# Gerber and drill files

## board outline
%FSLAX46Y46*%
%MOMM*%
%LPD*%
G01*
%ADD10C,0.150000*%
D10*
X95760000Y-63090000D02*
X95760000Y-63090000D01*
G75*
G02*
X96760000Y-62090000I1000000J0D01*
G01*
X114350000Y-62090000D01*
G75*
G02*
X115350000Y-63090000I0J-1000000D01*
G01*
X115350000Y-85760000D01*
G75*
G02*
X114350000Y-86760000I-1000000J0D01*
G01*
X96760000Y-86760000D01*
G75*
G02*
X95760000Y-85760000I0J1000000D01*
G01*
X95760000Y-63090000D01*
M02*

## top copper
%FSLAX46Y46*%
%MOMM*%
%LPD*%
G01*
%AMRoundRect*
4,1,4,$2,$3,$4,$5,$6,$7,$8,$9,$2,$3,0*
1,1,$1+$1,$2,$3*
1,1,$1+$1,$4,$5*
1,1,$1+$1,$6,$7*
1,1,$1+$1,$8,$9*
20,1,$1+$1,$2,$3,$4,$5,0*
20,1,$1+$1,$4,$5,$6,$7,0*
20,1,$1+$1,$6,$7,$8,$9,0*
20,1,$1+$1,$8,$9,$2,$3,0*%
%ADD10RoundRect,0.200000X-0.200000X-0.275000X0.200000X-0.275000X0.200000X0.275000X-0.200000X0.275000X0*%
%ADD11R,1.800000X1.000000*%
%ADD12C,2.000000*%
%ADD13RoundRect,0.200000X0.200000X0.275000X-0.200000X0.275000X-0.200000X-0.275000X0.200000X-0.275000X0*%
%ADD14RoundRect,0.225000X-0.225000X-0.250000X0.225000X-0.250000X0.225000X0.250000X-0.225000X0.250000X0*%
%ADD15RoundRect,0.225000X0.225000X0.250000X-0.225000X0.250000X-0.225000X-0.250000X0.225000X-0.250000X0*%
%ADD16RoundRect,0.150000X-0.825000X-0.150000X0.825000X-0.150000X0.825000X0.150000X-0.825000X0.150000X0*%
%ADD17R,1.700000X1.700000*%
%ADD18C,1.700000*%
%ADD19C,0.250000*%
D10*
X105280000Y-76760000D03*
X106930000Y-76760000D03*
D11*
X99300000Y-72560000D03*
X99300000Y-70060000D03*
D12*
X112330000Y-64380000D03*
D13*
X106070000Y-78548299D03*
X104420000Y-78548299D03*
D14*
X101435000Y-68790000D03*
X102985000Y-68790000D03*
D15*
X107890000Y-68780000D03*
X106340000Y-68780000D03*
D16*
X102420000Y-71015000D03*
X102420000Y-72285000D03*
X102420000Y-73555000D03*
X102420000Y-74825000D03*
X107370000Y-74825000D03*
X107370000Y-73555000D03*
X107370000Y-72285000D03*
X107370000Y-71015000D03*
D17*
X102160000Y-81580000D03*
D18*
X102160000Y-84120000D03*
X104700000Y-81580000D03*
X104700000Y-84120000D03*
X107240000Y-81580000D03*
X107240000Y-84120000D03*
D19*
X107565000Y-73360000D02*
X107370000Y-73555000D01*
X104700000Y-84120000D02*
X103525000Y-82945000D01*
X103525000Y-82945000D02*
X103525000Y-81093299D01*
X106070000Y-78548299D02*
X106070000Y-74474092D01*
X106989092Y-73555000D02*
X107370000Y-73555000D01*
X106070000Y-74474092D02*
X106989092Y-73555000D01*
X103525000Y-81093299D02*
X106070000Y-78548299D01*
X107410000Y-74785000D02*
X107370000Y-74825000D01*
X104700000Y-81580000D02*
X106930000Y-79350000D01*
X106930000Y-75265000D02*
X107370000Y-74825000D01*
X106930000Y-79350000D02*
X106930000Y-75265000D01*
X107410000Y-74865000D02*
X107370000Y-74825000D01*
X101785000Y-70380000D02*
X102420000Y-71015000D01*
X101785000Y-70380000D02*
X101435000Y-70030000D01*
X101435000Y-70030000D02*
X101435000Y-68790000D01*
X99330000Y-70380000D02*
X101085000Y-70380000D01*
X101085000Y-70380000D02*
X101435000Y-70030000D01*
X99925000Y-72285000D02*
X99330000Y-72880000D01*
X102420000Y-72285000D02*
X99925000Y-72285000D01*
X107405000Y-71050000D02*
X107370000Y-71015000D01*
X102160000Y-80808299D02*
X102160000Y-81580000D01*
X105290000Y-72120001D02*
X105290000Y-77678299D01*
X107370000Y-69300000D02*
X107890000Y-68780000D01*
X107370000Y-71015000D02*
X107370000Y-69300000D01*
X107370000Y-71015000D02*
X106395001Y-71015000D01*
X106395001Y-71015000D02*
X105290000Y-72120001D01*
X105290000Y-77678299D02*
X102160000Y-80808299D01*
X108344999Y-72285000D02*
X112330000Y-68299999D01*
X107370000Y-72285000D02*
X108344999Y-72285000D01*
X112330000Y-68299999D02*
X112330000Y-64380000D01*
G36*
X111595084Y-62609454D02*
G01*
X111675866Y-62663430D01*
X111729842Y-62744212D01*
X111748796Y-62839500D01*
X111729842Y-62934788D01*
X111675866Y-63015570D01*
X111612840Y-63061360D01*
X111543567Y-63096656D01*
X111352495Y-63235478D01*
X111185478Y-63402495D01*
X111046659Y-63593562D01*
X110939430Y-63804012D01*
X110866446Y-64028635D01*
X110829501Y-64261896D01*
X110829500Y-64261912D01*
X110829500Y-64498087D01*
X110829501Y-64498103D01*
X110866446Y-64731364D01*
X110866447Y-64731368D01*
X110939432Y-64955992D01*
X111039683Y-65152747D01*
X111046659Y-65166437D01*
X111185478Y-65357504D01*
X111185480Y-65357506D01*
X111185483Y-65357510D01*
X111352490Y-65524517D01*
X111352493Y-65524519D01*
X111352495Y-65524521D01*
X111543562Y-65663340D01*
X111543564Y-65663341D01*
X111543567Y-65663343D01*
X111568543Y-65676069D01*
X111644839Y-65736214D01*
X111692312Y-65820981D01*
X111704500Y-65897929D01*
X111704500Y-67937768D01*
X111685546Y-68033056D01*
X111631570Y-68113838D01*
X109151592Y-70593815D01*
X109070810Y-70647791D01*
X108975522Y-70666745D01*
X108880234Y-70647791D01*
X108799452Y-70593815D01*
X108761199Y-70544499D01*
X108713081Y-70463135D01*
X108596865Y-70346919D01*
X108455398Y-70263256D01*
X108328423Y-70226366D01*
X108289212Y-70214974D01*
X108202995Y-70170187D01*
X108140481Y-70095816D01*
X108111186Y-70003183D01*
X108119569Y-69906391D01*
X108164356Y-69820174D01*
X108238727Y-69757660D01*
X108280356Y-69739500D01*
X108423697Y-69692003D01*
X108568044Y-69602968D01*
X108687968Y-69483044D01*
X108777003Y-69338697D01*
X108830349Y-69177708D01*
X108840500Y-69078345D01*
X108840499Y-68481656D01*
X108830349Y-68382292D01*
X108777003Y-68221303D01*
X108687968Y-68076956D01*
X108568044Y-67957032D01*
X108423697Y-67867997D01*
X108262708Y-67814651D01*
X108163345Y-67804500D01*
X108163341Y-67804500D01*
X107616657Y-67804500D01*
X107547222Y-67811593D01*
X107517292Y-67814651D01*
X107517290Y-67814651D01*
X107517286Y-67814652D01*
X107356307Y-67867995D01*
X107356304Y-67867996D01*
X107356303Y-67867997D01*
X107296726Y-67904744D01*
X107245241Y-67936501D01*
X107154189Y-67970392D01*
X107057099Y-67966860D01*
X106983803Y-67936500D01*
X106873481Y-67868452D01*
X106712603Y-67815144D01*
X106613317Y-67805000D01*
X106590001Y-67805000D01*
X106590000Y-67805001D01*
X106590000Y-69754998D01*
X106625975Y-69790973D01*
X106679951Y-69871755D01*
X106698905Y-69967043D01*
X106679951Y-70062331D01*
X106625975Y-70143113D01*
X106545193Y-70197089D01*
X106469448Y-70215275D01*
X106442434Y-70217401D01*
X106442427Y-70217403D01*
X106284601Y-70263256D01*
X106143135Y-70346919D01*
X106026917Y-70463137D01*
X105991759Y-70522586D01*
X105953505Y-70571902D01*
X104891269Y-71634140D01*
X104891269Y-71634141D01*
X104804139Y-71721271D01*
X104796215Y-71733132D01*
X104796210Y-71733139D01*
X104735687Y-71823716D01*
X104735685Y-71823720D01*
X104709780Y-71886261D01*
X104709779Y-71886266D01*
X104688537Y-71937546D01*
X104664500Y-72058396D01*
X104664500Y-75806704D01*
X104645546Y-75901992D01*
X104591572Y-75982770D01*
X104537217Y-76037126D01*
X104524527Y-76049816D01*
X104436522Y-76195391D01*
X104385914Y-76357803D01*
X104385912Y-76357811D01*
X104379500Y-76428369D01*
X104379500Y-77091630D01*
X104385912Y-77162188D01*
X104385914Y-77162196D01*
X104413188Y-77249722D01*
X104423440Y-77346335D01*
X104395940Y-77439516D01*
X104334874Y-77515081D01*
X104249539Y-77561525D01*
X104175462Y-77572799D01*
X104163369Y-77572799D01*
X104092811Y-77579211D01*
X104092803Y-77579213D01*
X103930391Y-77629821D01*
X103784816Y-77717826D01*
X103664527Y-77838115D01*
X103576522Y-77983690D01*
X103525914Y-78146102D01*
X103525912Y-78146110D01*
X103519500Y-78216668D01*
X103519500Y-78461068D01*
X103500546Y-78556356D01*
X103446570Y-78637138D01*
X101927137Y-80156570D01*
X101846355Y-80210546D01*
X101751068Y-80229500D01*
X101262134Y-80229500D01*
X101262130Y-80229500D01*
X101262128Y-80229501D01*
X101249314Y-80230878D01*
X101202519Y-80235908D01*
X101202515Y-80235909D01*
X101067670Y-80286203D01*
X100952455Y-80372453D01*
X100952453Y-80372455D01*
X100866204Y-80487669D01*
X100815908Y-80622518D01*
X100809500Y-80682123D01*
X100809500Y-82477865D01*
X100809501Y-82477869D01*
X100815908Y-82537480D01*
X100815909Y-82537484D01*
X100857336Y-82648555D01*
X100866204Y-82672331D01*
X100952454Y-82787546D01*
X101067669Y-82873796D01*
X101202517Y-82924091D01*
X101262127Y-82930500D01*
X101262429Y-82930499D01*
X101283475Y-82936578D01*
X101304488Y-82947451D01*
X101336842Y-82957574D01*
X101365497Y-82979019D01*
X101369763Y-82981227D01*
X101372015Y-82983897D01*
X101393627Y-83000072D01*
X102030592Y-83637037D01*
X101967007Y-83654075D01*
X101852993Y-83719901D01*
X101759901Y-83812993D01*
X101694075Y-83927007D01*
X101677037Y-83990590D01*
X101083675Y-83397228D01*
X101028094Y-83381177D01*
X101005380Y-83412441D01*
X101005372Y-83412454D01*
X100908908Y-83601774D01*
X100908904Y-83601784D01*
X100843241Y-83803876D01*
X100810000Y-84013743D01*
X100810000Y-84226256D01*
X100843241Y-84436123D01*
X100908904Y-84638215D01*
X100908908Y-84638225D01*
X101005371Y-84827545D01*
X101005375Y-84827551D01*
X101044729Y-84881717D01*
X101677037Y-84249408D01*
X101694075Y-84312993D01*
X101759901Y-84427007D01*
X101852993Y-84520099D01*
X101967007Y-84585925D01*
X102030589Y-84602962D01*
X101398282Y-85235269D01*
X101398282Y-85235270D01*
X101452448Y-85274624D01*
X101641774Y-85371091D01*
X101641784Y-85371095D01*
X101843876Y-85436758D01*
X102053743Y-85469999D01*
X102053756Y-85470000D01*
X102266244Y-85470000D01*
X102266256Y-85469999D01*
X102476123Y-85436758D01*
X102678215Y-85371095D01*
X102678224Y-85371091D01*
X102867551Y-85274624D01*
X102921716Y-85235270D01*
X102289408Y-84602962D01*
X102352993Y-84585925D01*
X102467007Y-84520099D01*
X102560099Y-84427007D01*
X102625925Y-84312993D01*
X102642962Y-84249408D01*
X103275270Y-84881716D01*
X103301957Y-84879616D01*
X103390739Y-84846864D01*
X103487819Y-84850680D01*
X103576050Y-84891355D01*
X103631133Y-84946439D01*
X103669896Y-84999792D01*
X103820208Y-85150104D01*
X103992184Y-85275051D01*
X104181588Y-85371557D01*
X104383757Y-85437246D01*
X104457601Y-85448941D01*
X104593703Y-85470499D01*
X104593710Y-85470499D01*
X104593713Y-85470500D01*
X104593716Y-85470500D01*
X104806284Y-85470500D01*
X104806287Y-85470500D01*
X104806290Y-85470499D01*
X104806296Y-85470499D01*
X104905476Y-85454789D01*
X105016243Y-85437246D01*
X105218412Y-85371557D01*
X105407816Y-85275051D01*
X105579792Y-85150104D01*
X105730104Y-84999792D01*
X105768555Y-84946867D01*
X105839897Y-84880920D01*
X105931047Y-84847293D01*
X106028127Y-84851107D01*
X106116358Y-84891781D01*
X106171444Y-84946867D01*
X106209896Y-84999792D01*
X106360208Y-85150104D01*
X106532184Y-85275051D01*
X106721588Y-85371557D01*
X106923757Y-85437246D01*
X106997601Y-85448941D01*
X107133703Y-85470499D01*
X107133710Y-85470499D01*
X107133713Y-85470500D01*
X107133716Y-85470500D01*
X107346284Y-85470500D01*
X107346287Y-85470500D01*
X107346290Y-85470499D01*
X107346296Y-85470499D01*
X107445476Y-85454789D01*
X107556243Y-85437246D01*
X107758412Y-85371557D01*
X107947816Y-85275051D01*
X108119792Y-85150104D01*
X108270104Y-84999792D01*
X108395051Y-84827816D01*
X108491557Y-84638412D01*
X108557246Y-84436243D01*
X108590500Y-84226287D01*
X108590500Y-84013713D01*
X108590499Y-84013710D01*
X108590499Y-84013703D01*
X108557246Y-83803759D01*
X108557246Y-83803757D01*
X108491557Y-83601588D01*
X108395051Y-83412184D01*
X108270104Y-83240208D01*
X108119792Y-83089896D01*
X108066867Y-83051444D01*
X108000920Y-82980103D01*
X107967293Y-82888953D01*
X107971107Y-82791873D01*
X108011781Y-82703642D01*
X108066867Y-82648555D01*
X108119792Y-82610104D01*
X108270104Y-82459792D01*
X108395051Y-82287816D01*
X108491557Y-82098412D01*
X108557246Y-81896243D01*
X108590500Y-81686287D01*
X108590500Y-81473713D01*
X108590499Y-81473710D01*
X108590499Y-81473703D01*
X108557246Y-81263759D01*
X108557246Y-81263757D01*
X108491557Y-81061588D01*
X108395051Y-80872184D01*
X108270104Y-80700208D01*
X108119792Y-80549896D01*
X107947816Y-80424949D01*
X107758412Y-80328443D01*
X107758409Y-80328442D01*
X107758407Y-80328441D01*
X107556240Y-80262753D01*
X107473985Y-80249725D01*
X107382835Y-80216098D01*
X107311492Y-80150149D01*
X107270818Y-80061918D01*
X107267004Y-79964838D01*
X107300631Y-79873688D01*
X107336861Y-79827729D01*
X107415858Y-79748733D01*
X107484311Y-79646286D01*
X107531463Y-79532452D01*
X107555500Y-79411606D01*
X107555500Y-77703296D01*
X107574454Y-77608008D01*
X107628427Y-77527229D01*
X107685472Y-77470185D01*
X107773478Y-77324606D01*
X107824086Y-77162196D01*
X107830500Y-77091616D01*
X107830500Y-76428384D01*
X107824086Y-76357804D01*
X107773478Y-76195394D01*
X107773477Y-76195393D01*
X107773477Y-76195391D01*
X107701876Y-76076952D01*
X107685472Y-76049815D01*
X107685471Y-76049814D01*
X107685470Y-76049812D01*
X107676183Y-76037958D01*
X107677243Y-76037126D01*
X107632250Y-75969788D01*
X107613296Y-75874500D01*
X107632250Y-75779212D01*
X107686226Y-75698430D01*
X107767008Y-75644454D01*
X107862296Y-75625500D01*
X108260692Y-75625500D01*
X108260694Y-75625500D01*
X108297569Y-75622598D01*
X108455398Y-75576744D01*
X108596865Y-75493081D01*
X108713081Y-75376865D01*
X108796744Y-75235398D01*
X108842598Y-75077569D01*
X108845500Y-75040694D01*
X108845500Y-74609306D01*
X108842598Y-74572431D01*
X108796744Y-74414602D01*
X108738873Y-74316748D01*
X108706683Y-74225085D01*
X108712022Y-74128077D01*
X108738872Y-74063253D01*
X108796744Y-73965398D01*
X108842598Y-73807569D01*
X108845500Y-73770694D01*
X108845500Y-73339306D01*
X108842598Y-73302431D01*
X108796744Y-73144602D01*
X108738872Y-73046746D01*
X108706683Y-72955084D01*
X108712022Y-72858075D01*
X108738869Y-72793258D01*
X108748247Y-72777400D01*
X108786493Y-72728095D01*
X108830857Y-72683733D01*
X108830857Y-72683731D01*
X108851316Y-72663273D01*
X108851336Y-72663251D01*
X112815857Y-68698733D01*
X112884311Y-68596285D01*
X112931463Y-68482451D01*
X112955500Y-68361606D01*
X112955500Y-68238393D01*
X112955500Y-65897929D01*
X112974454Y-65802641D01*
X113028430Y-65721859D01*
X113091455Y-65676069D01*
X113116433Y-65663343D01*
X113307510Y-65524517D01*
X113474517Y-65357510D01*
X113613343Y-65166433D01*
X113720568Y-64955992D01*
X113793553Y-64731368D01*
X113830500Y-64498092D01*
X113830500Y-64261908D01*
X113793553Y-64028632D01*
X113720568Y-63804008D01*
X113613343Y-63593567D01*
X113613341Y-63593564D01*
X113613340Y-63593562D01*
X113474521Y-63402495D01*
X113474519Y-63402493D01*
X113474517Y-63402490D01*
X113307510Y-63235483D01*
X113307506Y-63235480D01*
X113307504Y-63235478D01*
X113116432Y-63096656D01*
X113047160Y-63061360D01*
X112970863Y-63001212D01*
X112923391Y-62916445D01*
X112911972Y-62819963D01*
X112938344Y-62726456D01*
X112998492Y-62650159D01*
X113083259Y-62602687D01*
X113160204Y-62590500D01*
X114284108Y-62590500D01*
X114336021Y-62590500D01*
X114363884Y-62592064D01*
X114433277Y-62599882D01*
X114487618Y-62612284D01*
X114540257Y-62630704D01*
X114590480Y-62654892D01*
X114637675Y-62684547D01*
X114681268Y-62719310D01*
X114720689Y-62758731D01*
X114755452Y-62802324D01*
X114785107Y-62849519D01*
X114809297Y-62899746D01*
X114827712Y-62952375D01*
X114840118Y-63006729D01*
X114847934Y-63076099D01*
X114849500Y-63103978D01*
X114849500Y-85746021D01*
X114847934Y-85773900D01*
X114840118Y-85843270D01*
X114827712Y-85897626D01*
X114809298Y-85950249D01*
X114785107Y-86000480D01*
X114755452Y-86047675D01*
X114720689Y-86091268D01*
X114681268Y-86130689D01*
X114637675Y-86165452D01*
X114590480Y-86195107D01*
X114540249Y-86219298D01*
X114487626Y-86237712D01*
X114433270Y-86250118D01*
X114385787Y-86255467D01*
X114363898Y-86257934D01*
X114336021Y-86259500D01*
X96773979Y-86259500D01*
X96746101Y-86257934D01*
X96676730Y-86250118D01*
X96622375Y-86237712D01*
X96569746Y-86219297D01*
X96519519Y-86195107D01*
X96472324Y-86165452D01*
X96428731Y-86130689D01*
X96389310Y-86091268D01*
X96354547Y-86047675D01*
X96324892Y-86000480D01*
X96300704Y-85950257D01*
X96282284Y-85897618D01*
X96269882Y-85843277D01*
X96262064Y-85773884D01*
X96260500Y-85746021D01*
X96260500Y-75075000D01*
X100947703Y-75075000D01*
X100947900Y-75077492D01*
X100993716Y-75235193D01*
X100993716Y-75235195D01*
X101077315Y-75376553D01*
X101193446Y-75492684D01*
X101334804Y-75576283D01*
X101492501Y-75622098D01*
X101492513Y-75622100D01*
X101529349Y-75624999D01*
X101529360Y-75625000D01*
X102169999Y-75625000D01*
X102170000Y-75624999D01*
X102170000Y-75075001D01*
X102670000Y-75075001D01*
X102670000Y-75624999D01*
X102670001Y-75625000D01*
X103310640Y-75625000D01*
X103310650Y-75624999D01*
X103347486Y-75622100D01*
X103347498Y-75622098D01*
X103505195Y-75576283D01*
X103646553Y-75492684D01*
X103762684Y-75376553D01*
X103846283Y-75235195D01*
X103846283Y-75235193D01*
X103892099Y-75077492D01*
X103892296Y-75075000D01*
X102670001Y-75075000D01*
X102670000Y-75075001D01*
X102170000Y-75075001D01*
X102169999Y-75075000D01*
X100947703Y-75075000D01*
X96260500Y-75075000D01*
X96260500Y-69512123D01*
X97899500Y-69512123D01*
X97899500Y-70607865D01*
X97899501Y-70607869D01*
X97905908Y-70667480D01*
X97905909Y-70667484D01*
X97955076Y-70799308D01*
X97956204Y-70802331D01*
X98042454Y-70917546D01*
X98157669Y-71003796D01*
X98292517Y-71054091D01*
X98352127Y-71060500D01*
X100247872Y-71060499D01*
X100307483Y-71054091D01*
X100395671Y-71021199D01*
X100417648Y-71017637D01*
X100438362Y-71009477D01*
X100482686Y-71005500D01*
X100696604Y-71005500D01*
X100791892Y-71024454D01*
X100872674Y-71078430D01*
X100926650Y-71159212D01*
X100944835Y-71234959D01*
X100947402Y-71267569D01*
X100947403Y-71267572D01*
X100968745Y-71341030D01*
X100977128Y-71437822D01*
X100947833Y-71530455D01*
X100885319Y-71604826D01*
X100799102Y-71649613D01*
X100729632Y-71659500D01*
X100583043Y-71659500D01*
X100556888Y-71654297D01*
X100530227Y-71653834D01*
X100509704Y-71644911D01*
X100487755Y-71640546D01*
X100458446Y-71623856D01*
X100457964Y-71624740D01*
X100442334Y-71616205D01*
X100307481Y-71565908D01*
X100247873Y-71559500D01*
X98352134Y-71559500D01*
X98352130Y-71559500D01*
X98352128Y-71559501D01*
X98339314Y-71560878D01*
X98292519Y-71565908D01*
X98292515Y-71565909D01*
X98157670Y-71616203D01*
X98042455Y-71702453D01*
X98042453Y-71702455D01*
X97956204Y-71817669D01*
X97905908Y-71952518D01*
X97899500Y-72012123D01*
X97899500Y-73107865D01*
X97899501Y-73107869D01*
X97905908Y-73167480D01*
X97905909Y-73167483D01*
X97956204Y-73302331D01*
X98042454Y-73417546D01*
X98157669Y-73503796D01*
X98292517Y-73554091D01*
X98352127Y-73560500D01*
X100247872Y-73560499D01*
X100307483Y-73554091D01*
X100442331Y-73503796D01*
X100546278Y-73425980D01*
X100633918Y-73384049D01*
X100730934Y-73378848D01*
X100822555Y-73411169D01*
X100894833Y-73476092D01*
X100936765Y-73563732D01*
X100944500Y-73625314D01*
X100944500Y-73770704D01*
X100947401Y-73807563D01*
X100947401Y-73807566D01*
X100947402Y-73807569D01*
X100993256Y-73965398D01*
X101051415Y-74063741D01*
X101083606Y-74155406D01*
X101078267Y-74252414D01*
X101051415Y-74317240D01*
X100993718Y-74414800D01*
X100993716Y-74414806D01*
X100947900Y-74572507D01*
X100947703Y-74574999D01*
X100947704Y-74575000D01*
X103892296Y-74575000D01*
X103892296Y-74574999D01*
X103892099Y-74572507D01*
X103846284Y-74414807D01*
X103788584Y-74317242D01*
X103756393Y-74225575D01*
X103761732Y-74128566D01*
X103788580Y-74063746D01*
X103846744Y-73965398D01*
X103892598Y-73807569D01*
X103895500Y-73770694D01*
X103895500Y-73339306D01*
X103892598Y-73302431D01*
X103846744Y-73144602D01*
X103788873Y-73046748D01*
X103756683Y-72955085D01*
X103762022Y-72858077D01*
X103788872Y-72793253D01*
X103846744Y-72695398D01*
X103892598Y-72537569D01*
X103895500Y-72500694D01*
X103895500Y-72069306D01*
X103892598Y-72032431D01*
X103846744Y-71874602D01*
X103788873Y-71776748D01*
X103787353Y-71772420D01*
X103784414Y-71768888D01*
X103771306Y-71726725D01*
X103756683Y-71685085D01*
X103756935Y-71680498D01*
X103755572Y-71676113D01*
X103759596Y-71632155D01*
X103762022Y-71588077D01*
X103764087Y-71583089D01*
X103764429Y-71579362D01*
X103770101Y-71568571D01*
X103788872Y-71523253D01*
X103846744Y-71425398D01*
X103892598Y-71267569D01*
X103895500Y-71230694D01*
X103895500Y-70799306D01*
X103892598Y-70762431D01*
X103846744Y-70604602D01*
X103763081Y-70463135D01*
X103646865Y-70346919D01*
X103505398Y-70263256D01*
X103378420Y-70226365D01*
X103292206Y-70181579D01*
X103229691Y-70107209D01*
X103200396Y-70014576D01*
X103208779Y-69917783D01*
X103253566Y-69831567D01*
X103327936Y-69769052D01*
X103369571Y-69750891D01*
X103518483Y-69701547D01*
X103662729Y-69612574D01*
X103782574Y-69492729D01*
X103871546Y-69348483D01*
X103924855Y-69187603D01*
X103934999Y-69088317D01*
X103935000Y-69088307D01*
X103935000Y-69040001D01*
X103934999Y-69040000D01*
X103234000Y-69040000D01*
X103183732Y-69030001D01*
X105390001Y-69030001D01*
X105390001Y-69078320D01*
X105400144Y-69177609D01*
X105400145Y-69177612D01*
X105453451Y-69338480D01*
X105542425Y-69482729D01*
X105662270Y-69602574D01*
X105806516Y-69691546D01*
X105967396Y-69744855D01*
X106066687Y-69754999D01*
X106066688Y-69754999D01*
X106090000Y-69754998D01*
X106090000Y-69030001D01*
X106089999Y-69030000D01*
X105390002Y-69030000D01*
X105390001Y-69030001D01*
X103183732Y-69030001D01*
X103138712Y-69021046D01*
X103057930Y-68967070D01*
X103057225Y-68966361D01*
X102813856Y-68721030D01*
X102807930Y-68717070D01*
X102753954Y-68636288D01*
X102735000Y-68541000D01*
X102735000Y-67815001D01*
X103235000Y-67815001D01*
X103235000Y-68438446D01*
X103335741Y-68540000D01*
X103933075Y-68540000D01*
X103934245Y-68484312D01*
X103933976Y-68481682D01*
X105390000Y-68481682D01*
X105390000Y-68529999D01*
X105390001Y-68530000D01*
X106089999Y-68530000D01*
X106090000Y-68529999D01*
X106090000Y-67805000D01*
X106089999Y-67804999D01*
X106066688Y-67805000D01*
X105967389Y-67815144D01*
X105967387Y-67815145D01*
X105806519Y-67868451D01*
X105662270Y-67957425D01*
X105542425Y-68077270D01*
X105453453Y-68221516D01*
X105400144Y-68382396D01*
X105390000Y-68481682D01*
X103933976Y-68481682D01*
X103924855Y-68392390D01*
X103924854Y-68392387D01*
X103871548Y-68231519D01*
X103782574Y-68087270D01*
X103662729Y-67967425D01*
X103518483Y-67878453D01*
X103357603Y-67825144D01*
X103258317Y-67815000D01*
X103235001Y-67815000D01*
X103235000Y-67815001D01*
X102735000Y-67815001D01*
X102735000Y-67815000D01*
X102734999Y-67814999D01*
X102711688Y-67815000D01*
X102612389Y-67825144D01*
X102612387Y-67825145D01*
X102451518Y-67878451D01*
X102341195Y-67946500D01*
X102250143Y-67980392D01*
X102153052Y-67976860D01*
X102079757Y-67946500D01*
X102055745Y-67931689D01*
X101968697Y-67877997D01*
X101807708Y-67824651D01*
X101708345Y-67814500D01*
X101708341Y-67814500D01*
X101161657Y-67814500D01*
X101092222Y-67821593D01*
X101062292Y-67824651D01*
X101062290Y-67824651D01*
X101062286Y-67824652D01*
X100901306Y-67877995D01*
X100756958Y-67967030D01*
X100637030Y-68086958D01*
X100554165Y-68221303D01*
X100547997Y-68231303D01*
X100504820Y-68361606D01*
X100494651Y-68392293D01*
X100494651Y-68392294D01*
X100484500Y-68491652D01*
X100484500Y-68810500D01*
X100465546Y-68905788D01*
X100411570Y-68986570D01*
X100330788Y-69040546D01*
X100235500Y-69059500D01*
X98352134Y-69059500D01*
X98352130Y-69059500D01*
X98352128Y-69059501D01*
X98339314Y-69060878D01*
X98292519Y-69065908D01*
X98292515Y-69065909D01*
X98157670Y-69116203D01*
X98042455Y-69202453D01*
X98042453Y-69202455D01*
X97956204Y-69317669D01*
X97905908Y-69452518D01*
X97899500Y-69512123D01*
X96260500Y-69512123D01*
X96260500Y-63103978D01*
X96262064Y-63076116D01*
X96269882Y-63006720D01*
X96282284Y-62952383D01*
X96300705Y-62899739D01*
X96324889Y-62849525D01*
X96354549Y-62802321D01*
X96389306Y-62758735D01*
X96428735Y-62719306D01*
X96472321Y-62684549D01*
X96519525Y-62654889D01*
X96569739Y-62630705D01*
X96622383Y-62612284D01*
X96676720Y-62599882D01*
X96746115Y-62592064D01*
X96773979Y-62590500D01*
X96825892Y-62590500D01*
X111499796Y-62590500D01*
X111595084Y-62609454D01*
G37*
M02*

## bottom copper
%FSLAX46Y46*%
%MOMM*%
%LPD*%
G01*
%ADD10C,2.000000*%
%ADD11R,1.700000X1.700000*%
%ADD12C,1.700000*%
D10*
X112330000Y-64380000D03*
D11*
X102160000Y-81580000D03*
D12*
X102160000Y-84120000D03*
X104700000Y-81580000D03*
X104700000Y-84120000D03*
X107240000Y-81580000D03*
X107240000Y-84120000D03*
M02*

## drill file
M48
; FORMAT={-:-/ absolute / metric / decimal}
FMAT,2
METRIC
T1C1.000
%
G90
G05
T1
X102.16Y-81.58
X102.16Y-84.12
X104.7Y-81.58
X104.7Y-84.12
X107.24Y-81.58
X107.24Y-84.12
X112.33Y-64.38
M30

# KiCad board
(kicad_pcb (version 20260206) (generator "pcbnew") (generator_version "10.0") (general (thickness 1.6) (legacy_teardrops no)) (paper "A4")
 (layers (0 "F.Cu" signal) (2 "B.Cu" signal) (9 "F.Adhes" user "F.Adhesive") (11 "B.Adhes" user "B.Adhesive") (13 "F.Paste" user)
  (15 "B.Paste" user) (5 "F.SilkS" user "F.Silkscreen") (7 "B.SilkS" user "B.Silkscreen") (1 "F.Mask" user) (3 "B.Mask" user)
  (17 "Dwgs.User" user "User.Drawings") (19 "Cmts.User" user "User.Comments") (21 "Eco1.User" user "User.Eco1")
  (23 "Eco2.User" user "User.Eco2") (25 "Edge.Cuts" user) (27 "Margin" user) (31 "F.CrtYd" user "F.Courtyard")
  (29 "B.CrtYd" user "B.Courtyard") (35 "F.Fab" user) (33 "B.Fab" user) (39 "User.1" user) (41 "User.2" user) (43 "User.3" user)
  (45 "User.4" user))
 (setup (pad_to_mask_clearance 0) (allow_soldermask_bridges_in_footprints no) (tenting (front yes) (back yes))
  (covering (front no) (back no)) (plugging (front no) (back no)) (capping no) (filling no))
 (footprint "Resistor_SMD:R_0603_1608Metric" (layer "F.Cu") (at 106.105 76.76)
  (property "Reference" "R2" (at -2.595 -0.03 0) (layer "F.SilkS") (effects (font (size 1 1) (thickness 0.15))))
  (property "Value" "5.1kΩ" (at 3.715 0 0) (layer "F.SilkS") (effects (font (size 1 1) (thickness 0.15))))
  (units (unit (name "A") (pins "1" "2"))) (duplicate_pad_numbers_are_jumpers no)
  (pad "1" smd roundrect (at -0.825 0) (size 0.8 0.95) (layers "F.Cu" "F.Mask" "F.Paste") (roundrect_rratio 0.25) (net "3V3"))
  (pad "2" smd roundrect (at 0.825 0) (size 0.8 0.95) (layers "F.Cu" "F.Mask" "F.Paste") (roundrect_rratio 0.25) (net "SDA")))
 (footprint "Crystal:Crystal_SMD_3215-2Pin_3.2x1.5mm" (layer "F.Cu") (at 99.3 71.31 -90)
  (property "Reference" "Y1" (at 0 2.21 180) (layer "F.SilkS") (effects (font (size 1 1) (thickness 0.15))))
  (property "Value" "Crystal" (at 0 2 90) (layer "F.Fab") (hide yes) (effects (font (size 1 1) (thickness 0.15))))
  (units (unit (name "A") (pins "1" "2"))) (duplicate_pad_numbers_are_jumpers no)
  (pad "1" smd rect (at 1.25 0 270) (size 1 1.8) (layers "F.Cu" "F.Mask" "F.Paste") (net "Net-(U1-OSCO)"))
  (pad "2" smd rect (at -1.25 0 270) (size 1 1.8) (layers "F.Cu" "F.Mask" "F.Paste") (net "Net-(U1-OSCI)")))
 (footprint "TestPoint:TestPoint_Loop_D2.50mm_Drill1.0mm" (layer "F.Cu") (at 112.33 64.38)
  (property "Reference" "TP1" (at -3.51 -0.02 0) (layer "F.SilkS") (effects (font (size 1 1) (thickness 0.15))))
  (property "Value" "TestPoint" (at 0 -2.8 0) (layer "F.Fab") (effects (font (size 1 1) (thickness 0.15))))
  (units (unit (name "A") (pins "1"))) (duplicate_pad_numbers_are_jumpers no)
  (pad "1" thru_hole circle (at 0 0) (size 2 2) (drill 1) (layers "*.Cu" "*.Mask") (remove_unused_layers no) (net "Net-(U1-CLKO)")))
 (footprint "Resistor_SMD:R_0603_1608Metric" (layer "F.Cu") (at 105.245 78.548299 180)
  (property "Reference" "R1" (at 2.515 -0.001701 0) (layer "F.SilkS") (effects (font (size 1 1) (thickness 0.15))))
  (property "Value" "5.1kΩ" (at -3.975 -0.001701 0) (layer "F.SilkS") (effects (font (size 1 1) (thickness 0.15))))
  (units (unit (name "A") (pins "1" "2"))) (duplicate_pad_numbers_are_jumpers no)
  (pad "1" smd roundrect (at -0.825 0 180) (size 0.8 0.95) (layers "F.Cu" "F.Mask" "F.Paste") (roundrect_rratio 0.25) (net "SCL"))
  (pad "2" smd roundrect (at 0.825 0 180) (size 0.8 0.95) (layers "F.Cu" "F.Mask" "F.Paste") (roundrect_rratio 0.25) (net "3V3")))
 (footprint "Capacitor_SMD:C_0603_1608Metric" (layer "F.Cu") (at 102.21 68.79)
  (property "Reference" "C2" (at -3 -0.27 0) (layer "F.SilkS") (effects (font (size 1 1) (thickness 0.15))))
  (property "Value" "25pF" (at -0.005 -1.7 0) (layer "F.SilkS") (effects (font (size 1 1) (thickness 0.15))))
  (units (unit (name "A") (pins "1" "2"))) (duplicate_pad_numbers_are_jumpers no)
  (pad "1" smd roundrect (at -0.775 0) (size 0.9 0.95) (layers "F.Cu" "F.Mask" "F.Paste") (roundrect_rratio 0.25) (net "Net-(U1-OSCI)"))
  (pad "2" smd roundrect (at 0.775 0) (size 0.9 0.95) (layers "F.Cu" "F.Mask" "F.Paste") (roundrect_rratio 0.25) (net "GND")))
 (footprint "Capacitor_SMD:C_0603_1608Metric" (layer "F.Cu") (at 107.115 68.78 180)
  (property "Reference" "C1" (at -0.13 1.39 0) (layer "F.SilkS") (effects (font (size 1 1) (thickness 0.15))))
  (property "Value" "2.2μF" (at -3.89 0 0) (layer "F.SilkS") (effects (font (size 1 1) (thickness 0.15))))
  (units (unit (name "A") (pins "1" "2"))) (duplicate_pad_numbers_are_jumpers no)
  (pad "1" smd roundrect (at -0.775 0 180) (size 0.9 0.95) (layers "F.Cu" "F.Mask" "F.Paste") (roundrect_rratio 0.25) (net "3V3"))
  (pad "2" smd roundrect (at 0.775 0 180) (size 0.9 0.95) (layers "F.Cu" "F.Mask" "F.Paste") (roundrect_rratio 0.25) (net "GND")))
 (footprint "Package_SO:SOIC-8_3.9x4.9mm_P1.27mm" (layer "F.Cu") (at 104.895 72.92)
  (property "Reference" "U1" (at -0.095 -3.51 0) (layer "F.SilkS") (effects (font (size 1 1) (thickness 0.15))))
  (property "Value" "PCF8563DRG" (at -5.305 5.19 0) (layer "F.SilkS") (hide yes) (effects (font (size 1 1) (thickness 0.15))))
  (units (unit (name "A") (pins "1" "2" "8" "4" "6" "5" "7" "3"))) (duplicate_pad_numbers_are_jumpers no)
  (pad "1" smd roundrect (at -2.475 -1.905) (size 1.95 0.6) (layers "F.Cu" "F.Mask" "F.Paste") (roundrect_rratio 0.25) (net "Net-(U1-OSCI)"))
  (pad "2" smd roundrect (at -2.475 -0.635) (size 1.95 0.6) (layers "F.Cu" "F.Mask" "F.Paste") (roundrect_rratio 0.25) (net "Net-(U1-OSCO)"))
  (pad "3" smd roundrect (at -2.475 0.635) (size 1.95 0.6) (layers "F.Cu" "F.Mask" "F.Paste") (roundrect_rratio 0.25)
   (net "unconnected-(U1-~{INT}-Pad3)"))
  (pad "4" smd roundrect (at -2.475 1.905) (size 1.95 0.6) (layers "F.Cu" "F.Mask" "F.Paste") (roundrect_rratio 0.25) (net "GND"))
  (pad "5" smd roundrect (at 2.475 1.905) (size 1.95 0.6) (layers "F.Cu" "F.Mask" "F.Paste") (roundrect_rratio 0.25) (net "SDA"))
  (pad "6" smd roundrect (at 2.475 0.635) (size 1.95 0.6) (layers "F.Cu" "F.Mask" "F.Paste") (roundrect_rratio 0.25) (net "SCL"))
  (pad "7" smd roundrect (at 2.475 -0.635) (size 1.95 0.6) (layers "F.Cu" "F.Mask" "F.Paste") (roundrect_rratio 0.25) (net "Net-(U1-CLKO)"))
  (pad "8" smd roundrect (at 2.475 -1.905) (size 1.95 0.6) (layers "F.Cu" "F.Mask" "F.Paste") (roundrect_rratio 0.25) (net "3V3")))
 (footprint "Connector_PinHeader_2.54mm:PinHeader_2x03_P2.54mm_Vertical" (layer "B.Cu") (at 102.16 81.58 -90)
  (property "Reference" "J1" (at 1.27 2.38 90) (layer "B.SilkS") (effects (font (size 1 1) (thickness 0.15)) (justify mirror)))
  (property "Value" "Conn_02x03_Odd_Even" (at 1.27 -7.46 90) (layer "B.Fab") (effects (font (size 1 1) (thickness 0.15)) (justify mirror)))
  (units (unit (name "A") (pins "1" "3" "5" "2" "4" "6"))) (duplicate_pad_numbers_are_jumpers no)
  (pad "1" thru_hole rect (at 0 0 270) (size 1.7 1.7) (drill 1) (layers "*.Cu" "*.Mask") (remove_unused_layers no) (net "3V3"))
  (pad "2" thru_hole circle (at 2.54 0 270) (size 1.7 1.7) (drill 1) (layers "*.Cu" "*.Mask") (remove_unused_layers no) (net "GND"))
  (pad "3" thru_hole circle (at 0 -2.54 270) (size 1.7 1.7) (drill 1) (layers "*.Cu" "*.Mask") (remove_unused_layers no) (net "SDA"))
  (pad "4" thru_hole circle (at 2.54 -2.54 270) (size 1.7 1.7) (drill 1) (layers "*.Cu" "*.Mask") (remove_unused_layers no) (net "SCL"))
  (pad "5" thru_hole circle (at 0 -5.08 270) (size 1.7 1.7) (drill 1) (layers "*.Cu" "*.Mask") (remove_unused_layers no)
   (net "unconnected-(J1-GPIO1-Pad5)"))
  (pad "6" thru_hole circle (at 2.54 -5.08 270) (size 1.7 1.7) (drill 1) (layers "*.Cu" "*.Mask") (remove_unused_layers no)
   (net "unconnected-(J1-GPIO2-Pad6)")))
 (gr_rect (start 95.76 62.09) (end 115.35 86.76) (radius 1) (stroke (width 0.15) (type solid)) (fill no) (layer "Edge.Cuts"))
 (segment (start 107.565 73.36) (end 107.37 73.555) (width 0.25) (layer "F.Cu") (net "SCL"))
 (segment (start 104.7 84.12) (end 103.525 82.945) (width 0.25) (layer "F.Cu") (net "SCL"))
 (segment (start 103.525 82.945) (end 103.525 81.093299) (width 0.25) (layer "F.Cu") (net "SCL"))
 (segment (start 106.07 78.548299) (end 106.07 74.474092) (width 0.25) (layer "F.Cu") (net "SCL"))
 (segment (start 106.989092 73.555) (end 107.37 73.555) (width 0.25) (layer "F.Cu") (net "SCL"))
 (segment (start 106.07 74.474092) (end 106.989092 73.555) (width 0.25) (layer "F.Cu") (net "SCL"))
 (segment (start 103.525 81.093299) (end 106.07 78.548299) (width 0.25) (layer "F.Cu") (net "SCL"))
 (segment (start 107.41 74.785) (end 107.37 74.825) (width 0.25) (layer "F.Cu") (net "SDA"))
 (segment (start 104.7 81.58) (end 106.93 79.35) (width 0.25) (layer "F.Cu") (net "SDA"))
 (segment (start 106.93 75.265) (end 107.37 74.825) (width 0.25) (layer "F.Cu") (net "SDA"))
 (segment (start 106.93 79.35) (end 106.93 75.265) (width 0.25) (layer "F.Cu") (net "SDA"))
 (segment (start 107.41 74.865) (end 107.37 74.825) (width 0.25) (layer "F.Cu") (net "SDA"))
 (segment (start 101.785 70.38) (end 102.42 71.015) (width 0.25) (layer "F.Cu") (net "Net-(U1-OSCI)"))
 (segment (start 101.785 70.38) (end 101.435 70.03) (width 0.25) (layer "F.Cu") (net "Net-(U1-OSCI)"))
 (segment (start 101.435 70.03) (end 101.435 68.79) (width 0.25) (layer "F.Cu") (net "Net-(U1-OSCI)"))
 (segment (start 99.33 70.38) (end 101.085 70.38) (width 0.25) (layer "F.Cu") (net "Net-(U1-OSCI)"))
 (segment (start 101.085 70.38) (end 101.435 70.03) (width 0.25) (layer "F.Cu") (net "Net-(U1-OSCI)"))
 (segment (start 99.925 72.285) (end 99.33 72.88) (width 0.25) (layer "F.Cu") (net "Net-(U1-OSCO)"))
 (segment (start 102.42 72.285) (end 99.925 72.285) (width 0.25) (layer "F.Cu") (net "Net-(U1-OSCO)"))
 (segment (start 107.405 71.05) (end 107.37 71.015) (width 0.25) (layer "F.Cu") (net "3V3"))
 (segment (start 102.16 80.808299) (end 102.16 81.58) (width 0.25) (layer "F.Cu") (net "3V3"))
 (segment (start 105.29 72.120001) (end 105.29 77.678299) (width 0.25) (layer "F.Cu") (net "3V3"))
 (segment (start 107.37 69.3) (end 107.89 68.78) (width 0.25) (layer "F.Cu") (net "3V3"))
 (segment (start 107.37 71.015) (end 107.37 69.3) (width 0.25) (layer "F.Cu") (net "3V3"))
 (segment (start 107.37 71.015) (end 106.395001 71.015) (width 0.25) (layer "F.Cu") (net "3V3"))
 (segment (start 106.395001 71.015) (end 105.29 72.120001) (width 0.25) (layer "F.Cu") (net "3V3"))
 (segment (start 105.29 77.678299) (end 102.16 80.808299) (width 0.25) (layer "F.Cu") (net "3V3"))
 (segment (start 108.344999 72.285) (end 112.33 68.299999) (width 0.25) (layer "F.Cu") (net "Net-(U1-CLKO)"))
 (segment (start 107.37 72.285) (end 108.344999 72.285) (width 0.25) (layer "F.Cu") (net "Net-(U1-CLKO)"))
 (segment (start 112.33 68.299999) (end 112.33 64.38) (width 0.25) (layer "F.Cu") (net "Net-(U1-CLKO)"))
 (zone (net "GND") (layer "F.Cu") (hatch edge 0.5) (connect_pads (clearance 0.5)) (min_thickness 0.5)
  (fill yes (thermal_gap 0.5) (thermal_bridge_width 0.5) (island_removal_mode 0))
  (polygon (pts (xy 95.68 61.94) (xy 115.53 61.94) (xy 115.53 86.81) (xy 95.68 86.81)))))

